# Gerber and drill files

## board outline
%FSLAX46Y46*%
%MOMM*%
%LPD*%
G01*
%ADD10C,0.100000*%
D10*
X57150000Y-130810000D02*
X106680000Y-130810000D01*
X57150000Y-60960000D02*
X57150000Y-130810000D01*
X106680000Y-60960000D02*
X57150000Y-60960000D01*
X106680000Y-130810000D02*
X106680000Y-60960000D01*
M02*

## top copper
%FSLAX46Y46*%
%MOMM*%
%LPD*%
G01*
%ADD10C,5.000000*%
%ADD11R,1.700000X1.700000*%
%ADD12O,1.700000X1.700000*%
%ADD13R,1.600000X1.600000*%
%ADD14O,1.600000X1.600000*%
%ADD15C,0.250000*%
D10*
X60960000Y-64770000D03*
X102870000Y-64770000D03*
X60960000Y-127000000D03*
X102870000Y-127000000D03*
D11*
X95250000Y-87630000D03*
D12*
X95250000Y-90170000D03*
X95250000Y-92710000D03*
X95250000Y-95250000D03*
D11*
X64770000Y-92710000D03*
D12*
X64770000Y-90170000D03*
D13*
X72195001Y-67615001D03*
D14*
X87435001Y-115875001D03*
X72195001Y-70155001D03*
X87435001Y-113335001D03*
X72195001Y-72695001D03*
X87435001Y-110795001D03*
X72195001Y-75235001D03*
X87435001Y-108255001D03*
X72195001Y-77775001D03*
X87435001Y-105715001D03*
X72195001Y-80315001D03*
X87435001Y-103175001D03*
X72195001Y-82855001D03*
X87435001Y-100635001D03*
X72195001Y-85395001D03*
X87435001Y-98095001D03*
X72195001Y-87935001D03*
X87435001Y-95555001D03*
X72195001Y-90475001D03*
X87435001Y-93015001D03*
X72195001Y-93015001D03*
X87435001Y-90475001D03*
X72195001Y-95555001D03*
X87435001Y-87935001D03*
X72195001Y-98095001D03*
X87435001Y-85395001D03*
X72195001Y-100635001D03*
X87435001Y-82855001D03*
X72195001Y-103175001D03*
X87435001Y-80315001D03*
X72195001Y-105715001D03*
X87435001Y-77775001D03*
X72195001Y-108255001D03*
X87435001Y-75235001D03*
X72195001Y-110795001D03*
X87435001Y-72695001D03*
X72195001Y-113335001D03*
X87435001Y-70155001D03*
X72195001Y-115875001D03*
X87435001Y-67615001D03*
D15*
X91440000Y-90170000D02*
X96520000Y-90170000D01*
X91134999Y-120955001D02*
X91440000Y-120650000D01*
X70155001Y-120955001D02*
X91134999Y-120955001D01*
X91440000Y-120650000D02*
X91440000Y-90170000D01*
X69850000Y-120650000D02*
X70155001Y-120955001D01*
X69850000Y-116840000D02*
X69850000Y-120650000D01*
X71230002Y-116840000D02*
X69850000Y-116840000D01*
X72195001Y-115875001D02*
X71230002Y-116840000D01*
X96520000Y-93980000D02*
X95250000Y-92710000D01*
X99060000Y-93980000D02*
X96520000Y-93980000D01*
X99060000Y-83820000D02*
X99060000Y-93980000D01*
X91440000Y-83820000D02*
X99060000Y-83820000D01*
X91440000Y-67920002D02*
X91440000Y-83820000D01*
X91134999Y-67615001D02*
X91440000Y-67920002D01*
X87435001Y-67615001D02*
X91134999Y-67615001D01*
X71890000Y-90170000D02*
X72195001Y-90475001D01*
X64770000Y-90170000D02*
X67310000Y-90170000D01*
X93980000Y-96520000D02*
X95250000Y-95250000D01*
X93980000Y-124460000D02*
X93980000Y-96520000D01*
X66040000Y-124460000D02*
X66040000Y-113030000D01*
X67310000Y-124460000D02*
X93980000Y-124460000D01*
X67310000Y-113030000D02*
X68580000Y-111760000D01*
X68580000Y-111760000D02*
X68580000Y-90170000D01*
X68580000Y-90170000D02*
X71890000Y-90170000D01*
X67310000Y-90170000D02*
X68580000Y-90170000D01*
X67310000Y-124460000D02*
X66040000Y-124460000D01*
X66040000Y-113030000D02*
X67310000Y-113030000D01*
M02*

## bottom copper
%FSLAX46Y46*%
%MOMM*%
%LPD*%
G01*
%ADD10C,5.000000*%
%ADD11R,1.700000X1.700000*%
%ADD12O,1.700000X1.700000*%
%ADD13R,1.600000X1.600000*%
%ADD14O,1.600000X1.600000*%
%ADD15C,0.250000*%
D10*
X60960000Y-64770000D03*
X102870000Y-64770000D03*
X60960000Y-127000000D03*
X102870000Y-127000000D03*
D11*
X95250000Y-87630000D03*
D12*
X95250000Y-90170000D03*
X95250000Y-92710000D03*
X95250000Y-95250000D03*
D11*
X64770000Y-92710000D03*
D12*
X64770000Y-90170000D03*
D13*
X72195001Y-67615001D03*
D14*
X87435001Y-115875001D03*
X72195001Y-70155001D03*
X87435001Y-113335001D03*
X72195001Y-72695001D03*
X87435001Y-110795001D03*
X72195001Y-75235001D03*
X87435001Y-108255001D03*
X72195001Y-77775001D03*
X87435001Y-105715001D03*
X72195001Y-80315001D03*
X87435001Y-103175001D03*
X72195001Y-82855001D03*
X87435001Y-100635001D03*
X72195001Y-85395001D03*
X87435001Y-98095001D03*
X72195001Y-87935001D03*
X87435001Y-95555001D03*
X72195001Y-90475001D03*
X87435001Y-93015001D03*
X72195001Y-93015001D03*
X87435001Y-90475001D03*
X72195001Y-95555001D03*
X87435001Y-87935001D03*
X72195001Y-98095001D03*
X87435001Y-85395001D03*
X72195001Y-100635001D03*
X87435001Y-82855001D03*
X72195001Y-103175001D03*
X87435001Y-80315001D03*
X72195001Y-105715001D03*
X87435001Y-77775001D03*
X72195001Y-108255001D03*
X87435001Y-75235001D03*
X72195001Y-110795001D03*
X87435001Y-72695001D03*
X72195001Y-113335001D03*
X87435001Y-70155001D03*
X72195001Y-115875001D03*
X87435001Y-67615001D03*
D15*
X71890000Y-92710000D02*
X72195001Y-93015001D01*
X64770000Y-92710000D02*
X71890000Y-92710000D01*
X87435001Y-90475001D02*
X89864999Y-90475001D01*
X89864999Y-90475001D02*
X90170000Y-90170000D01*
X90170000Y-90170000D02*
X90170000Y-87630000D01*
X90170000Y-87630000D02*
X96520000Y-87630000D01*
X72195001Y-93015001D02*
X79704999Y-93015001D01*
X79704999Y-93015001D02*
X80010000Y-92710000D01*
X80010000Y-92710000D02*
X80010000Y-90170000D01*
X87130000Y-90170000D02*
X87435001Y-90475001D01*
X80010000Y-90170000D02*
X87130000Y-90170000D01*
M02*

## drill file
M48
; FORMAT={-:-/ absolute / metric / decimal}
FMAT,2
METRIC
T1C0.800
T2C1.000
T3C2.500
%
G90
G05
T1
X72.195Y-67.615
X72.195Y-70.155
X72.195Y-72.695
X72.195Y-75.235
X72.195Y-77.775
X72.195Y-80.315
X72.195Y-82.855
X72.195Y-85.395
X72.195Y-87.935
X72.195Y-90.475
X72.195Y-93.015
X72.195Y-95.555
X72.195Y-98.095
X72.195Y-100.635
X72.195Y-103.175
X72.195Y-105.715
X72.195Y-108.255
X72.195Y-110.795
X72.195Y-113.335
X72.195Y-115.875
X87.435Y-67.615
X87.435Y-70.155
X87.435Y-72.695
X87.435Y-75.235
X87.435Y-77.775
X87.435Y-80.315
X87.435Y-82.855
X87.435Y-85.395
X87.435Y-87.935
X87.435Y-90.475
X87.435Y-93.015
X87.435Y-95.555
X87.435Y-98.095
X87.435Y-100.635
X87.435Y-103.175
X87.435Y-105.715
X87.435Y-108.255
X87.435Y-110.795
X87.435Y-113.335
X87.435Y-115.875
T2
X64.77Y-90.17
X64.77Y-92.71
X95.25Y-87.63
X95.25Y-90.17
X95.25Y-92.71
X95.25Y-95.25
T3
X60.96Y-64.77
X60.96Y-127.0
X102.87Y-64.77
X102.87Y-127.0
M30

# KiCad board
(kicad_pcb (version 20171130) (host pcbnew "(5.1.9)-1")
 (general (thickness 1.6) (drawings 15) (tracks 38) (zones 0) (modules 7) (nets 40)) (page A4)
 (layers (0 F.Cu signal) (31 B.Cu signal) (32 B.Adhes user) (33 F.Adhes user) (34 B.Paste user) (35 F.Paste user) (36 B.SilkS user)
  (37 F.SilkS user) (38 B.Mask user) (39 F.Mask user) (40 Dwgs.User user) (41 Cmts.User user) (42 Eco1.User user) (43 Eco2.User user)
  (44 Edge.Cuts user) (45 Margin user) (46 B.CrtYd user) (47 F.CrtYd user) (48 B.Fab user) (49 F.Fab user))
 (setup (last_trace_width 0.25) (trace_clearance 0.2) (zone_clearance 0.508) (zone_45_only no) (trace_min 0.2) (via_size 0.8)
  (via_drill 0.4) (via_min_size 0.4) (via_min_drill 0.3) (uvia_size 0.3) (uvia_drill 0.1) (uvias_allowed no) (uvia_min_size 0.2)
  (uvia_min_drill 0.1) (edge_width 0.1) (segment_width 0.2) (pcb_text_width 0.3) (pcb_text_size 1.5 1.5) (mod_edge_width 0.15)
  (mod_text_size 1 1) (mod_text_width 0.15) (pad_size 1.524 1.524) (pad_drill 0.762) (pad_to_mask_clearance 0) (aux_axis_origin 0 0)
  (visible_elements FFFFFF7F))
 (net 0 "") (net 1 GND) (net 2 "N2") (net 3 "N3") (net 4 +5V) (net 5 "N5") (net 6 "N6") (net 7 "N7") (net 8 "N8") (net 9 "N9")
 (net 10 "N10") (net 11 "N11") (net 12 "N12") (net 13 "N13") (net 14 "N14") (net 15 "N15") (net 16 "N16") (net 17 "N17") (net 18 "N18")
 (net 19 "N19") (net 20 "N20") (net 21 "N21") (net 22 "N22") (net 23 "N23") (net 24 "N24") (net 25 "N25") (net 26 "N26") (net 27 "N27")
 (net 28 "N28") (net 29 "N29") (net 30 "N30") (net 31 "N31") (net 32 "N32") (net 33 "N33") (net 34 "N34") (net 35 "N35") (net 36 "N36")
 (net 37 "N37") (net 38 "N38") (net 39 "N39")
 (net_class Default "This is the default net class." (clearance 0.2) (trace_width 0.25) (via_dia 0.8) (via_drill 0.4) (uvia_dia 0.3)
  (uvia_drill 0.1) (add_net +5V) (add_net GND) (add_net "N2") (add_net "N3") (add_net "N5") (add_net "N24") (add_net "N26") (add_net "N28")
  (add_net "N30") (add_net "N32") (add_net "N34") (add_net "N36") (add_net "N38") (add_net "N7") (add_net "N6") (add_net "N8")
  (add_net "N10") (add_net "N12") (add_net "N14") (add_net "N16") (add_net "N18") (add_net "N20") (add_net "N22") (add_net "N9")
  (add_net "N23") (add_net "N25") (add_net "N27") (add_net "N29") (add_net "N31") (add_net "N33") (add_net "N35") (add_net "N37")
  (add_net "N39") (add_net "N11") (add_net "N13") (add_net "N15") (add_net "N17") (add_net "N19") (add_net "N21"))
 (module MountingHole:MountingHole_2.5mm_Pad (layer F.Cu) (at 60.96 64.77)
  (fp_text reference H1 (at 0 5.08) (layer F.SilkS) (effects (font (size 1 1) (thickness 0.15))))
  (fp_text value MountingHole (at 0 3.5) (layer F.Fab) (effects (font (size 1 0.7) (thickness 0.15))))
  (pad 1 thru_hole circle (at 0 0) (size 5 5) (drill 2.5) (layers *.Cu *.Mask)))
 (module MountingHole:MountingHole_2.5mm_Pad (layer F.Cu) (at 102.87 64.77)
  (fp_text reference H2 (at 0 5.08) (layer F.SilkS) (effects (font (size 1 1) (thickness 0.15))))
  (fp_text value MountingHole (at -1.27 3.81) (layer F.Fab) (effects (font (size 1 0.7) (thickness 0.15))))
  (pad 1 thru_hole circle (at 0 0) (size 5 5) (drill 2.5) (layers *.Cu *.Mask)))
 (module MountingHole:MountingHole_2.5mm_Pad (layer F.Cu) (at 60.96 127)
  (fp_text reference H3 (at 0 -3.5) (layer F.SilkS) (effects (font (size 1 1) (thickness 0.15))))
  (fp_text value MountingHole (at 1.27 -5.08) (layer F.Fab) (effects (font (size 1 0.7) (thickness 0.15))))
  (pad 1 thru_hole circle (at 0 0) (size 5 5) (drill 2.5) (layers *.Cu *.Mask)))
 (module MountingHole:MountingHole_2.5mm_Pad (layer F.Cu) (at 102.87 127)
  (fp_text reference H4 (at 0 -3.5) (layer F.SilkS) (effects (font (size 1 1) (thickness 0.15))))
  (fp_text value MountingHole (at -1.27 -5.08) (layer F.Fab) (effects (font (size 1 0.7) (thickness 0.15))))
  (pad 1 thru_hole circle (at 0 0) (size 5 5) (drill 2.5) (layers *.Cu *.Mask)))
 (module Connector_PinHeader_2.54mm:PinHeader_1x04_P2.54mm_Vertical (layer F.Cu) (at 95.25 87.63)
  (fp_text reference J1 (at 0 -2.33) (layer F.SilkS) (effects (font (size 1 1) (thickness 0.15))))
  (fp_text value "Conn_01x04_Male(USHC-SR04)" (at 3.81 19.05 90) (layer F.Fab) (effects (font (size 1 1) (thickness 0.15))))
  (pad 1 thru_hole rect (at 0 0) (size 1.7 1.7) (drill 1) (layers *.Cu *.Mask) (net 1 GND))
  (pad 2 thru_hole oval (at 0 2.54) (size 1.7 1.7) (drill 1) (layers *.Cu *.Mask) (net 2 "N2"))
  (pad 3 thru_hole oval (at 0 5.08) (size 1.7 1.7) (drill 1) (layers *.Cu *.Mask) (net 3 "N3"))
  (pad 4 thru_hole oval (at 0 7.62) (size 1.7 1.7) (drill 1) (layers *.Cu *.Mask) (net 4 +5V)))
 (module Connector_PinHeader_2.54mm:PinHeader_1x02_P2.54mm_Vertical (layer F.Cu) (at 64.77 92.71 180)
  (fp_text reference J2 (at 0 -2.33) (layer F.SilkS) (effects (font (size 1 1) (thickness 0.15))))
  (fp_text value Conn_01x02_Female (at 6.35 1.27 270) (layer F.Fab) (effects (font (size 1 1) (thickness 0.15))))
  (pad 1 thru_hole rect (at 0 0 180) (size 1.7 1.7) (drill 1) (layers *.Cu *.Mask) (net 1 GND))
  (pad 2 thru_hole oval (at 0 2.54 180) (size 1.7 1.7) (drill 1) (layers *.Cu *.Mask) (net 4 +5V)))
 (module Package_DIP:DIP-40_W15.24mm (layer F.Cu) (at 72.195001 67.615001)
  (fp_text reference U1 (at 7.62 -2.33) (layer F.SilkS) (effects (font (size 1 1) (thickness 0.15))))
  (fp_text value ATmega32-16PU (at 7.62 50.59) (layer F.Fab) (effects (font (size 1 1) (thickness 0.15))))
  (pad 1 thru_hole rect (at 0 0) (size 1.6 1.6) (drill 0.8) (layers *.Cu *.Mask) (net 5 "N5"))
  (pad 21 thru_hole oval (at 15.24 48.26) (size 1.6 1.6) (drill 0.8) (layers *.Cu *.Mask) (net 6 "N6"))
  (pad 2 thru_hole oval (at 0 2.54) (size 1.6 1.6) (drill 0.8) (layers *.Cu *.Mask) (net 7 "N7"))
  (pad 22 thru_hole oval (at 15.24 45.72) (size 1.6 1.6) (drill 0.8) (layers *.Cu *.Mask) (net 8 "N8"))
  (pad 3 thru_hole oval (at 0 5.08) (size 1.6 1.6) (drill 0.8) (layers *.Cu *.Mask) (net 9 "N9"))
  (pad 23 thru_hole oval (at 15.24 43.18) (size 1.6 1.6) (drill 0.8) (layers *.Cu *.Mask) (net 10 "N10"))
  (pad 4 thru_hole oval (at 0 7.62) (size 1.6 1.6) (drill 0.8) (layers *.Cu *.Mask) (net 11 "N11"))
  (pad 24 thru_hole oval (at 15.24 40.64) (size 1.6 1.6) (drill 0.8) (layers *.Cu *.Mask) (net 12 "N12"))
  (pad 5 thru_hole oval (at 0 10.16) (size 1.6 1.6) (drill 0.8) (layers *.Cu *.Mask) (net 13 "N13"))
  (pad 25 thru_hole oval (at 15.24 38.1) (size 1.6 1.6) (drill 0.8) (layers *.Cu *.Mask) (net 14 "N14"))
  (pad 6 thru_hole oval (at 0 12.7) (size 1.6 1.6) (drill 0.8) (layers *.Cu *.Mask) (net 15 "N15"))
  (pad 26 thru_hole oval (at 15.24 35.56) (size 1.6 1.6) (drill 0.8) (layers *.Cu *.Mask) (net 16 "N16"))
  (pad 7 thru_hole oval (at 0 15.24) (size 1.6 1.6) (drill 0.8) (layers *.Cu *.Mask) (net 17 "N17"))
  (pad 27 thru_hole oval (at 15.24 33.02) (size 1.6 1.6) (drill 0.8) (layers *.Cu *.Mask) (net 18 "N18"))
  (pad 8 thru_hole oval (at 0 17.78) (size 1.6 1.6) (drill 0.8) (layers *.Cu *.Mask) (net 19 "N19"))
  (pad 28 thru_hole oval (at 15.24 30.48) (size 1.6 1.6) (drill 0.8) (layers *.Cu *.Mask) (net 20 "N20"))
  (pad 9 thru_hole oval (at 0 20.32) (size 1.6 1.6) (drill 0.8) (layers *.Cu *.Mask) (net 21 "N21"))
  (pad 29 thru_hole oval (at 15.24 27.94) (size 1.6 1.6) (drill 0.8) (layers *.Cu *.Mask) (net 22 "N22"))
  (pad 10 thru_hole oval (at 0 22.86) (size 1.6 1.6) (drill 0.8) (layers *.Cu *.Mask) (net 4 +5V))
  (pad 30 thru_hole oval (at 15.24 25.4) (size 1.6 1.6) (drill 0.8) (layers *.Cu *.Mask) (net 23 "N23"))
  (pad 11 thru_hole oval (at 0 25.4) (size 1.6 1.6) (drill 0.8) (layers *.Cu *.Mask) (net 1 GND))
  (pad 31 thru_hole oval (at 15.24 22.86) (size 1.6 1.6) (drill 0.8) (layers *.Cu *.Mask) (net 1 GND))
  (pad 12 thru_hole oval (at 0 27.94) (size 1.6 1.6) (drill 0.8) (layers *.Cu *.Mask) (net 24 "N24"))
  (pad 32 thru_hole oval (at 15.24 20.32) (size 1.6 1.6) (drill 0.8) (layers *.Cu *.Mask) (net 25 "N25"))
  (pad 13 thru_hole oval (at 0 30.48) (size 1.6 1.6) (drill 0.8) (layers *.Cu *.Mask) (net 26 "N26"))
  (pad 33 thru_hole oval (at 15.24 17.78) (size 1.6 1.6) (drill 0.8) (layers *.Cu *.Mask) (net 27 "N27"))
  (pad 14 thru_hole oval (at 0 33.02) (size 1.6 1.6) (drill 0.8) (layers *.Cu *.Mask) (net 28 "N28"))
  (pad 34 thru_hole oval (at 15.24 15.24) (size 1.6 1.6) (drill 0.8) (layers *.Cu *.Mask) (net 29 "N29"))
  (pad 15 thru_hole oval (at 0 35.56) (size 1.6 1.6) (drill 0.8) (layers *.Cu *.Mask) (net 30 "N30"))
  (pad 35 thru_hole oval (at 15.24 12.7) (size 1.6 1.6) (drill 0.8) (layers *.Cu *.Mask) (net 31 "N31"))
  (pad 16 thru_hole oval (at 0 38.1) (size 1.6 1.6) (drill 0.8) (layers *.Cu *.Mask) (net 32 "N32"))
  (pad 36 thru_hole oval (at 15.24 10.16) (size 1.6 1.6) (drill 0.8) (layers *.Cu *.Mask) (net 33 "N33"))
  (pad 17 thru_hole oval (at 0 40.64) (size 1.6 1.6) (drill 0.8) (layers *.Cu *.Mask) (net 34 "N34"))
  (pad 37 thru_hole oval (at 15.24 7.62) (size 1.6 1.6) (drill 0.8) (layers *.Cu *.Mask) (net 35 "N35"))
  (pad 18 thru_hole oval (at 0 43.18) (size 1.6 1.6) (drill 0.8) (layers *.Cu *.Mask) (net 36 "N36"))
  (pad 38 thru_hole oval (at 15.24 5.08) (size 1.6 1.6) (drill 0.8) (layers *.Cu *.Mask) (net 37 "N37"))
  (pad 19 thru_hole oval (at 0 45.72) (size 1.6 1.6) (drill 0.8) (layers *.Cu *.Mask) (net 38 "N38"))
  (pad 39 thru_hole oval (at 15.24 2.54) (size 1.6 1.6) (drill 0.8) (layers *.Cu *.Mask) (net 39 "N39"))
  (pad 20 thru_hole oval (at 0 48.26) (size 1.6 1.6) (drill 0.8) (layers *.Cu *.Mask) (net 2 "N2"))
  (pad 40 thru_hole oval (at 15.24 0) (size 1.6 1.6) (drill 0.8) (layers *.Cu *.Mask) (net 3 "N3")))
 (gr_line (start 57.15 130.81) (end 106.68 130.81) (layer Edge.Cuts) (width 0.1))
 (gr_line (start 57.15 60.96) (end 57.15 130.81) (layer Edge.Cuts) (width 0.1))
 (gr_line (start 106.68 60.96) (end 57.15 60.96) (layer Edge.Cuts) (width 0.1))
 (gr_line (start 106.68 130.81) (end 106.68 60.96) (layer Edge.Cuts) (width 0.1))
 (segment (start 71.89 92.71) (end 72.195001 93.015001) (width 0.25) (layer B.Cu) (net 1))
 (segment (start 64.77 92.71) (end 71.89 92.71) (width 0.25) (layer B.Cu) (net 1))
 (segment (start 87.435001 90.475001) (end 89.864999 90.475001) (width 0.25) (layer B.Cu) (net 1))
 (segment (start 89.864999 90.475001) (end 90.17 90.17) (width 0.25) (layer B.Cu) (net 1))
 (segment (start 90.17 90.17) (end 90.17 87.63) (width 0.25) (layer B.Cu) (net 1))
 (segment (start 90.17 87.63) (end 96.52 87.63) (width 0.25) (layer B.Cu) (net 1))
 (segment (start 72.195001 93.015001) (end 79.704999 93.015001) (width 0.25) (layer B.Cu) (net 1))
 (segment (start 79.704999 93.015001) (end 80.01 92.71) (width 0.25) (layer B.Cu) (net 1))
 (segment (start 80.01 92.71) (end 80.01 90.17) (width 0.25) (layer B.Cu) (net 1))
 (segment (start 87.13 90.17) (end 87.435001 90.475001) (width 0.25) (layer B.Cu) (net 1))
 (segment (start 80.01 90.17) (end 87.13 90.17) (width 0.25) (layer B.Cu) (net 1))
 (segment (start 91.44 90.17) (end 96.52 90.17) (width 0.25) (layer F.Cu) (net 2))
 (segment (start 91.134999 120.955001) (end 91.44 120.65) (width 0.25) (layer F.Cu) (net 2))
 (segment (start 70.155001 120.955001) (end 91.134999 120.955001) (width 0.25) (layer F.Cu) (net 2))
 (segment (start 91.44 120.65) (end 91.44 90.17) (width 0.25) (layer F.Cu) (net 2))
 (segment (start 69.85 120.65) (end 70.155001 120.955001) (width 0.25) (layer F.Cu) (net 2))
 (segment (start 69.85 116.84) (end 69.85 120.65) (width 0.25) (layer F.Cu) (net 2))
 (segment (start 71.230002 116.84) (end 69.85 116.84) (width 0.25) (layer F.Cu) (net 2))
 (segment (start 72.195001 115.875001) (end 71.230002 116.84) (width 0.25) (layer F.Cu) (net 2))
 (segment (start 96.52 93.98) (end 95.25 92.71) (width 0.25) (layer F.Cu) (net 3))
 (segment (start 99.06 93.98) (end 96.52 93.98) (width 0.25) (layer F.Cu) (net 3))
 (segment (start 99.06 83.82) (end 99.06 93.98) (width 0.25) (layer F.Cu) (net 3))
 (segment (start 91.44 83.82) (end 99.06 83.82) (width 0.25) (layer F.Cu) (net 3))
 (segment (start 91.44 67.920002) (end 91.44 83.82) (width 0.25) (layer F.Cu) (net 3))
 (segment (start 91.134999 67.615001) (end 91.44 67.920002) (width 0.25) (layer F.Cu) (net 3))
 (segment (start 87.435001 67.615001) (end 91.134999 67.615001) (width 0.25) (layer F.Cu) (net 3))
 (segment (start 71.89 90.17) (end 72.195001 90.475001) (width 0.25) (layer F.Cu) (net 4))
 (segment (start 64.77 90.17) (end 67.31 90.17) (width 0.25) (layer F.Cu) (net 4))
 (segment (start 93.98 96.52) (end 95.25 95.25) (width 0.25) (layer F.Cu) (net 4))
 (segment (start 93.98 124.46) (end 93.98 96.52) (width 0.25) (layer F.Cu) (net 4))
 (segment (start 66.04 124.46) (end 66.04 113.03) (width 0.25) (layer F.Cu) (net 4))
 (segment (start 67.31 124.46) (end 93.98 124.46) (width 0.25) (layer F.Cu) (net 4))
 (segment (start 67.31 113.03) (end 68.58 111.76) (width 0.25) (layer F.Cu) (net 4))
 (segment (start 68.58 111.76) (end 68.58 90.17) (width 0.25) (layer F.Cu) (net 4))
 (segment (start 68.58 90.17) (end 71.89 90.17) (width 0.25) (layer F.Cu) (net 4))
 (segment (start 67.31 90.17) (end 68.58 90.17) (width 0.25) (layer F.Cu) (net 4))
 (segment (start 67.31 124.46) (end 66.04 124.46) (width 0.25) (layer F.Cu) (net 4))
 (segment (start 66.04 113.03) (end 67.31 113.03) (width 0.25) (layer F.Cu) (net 4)))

